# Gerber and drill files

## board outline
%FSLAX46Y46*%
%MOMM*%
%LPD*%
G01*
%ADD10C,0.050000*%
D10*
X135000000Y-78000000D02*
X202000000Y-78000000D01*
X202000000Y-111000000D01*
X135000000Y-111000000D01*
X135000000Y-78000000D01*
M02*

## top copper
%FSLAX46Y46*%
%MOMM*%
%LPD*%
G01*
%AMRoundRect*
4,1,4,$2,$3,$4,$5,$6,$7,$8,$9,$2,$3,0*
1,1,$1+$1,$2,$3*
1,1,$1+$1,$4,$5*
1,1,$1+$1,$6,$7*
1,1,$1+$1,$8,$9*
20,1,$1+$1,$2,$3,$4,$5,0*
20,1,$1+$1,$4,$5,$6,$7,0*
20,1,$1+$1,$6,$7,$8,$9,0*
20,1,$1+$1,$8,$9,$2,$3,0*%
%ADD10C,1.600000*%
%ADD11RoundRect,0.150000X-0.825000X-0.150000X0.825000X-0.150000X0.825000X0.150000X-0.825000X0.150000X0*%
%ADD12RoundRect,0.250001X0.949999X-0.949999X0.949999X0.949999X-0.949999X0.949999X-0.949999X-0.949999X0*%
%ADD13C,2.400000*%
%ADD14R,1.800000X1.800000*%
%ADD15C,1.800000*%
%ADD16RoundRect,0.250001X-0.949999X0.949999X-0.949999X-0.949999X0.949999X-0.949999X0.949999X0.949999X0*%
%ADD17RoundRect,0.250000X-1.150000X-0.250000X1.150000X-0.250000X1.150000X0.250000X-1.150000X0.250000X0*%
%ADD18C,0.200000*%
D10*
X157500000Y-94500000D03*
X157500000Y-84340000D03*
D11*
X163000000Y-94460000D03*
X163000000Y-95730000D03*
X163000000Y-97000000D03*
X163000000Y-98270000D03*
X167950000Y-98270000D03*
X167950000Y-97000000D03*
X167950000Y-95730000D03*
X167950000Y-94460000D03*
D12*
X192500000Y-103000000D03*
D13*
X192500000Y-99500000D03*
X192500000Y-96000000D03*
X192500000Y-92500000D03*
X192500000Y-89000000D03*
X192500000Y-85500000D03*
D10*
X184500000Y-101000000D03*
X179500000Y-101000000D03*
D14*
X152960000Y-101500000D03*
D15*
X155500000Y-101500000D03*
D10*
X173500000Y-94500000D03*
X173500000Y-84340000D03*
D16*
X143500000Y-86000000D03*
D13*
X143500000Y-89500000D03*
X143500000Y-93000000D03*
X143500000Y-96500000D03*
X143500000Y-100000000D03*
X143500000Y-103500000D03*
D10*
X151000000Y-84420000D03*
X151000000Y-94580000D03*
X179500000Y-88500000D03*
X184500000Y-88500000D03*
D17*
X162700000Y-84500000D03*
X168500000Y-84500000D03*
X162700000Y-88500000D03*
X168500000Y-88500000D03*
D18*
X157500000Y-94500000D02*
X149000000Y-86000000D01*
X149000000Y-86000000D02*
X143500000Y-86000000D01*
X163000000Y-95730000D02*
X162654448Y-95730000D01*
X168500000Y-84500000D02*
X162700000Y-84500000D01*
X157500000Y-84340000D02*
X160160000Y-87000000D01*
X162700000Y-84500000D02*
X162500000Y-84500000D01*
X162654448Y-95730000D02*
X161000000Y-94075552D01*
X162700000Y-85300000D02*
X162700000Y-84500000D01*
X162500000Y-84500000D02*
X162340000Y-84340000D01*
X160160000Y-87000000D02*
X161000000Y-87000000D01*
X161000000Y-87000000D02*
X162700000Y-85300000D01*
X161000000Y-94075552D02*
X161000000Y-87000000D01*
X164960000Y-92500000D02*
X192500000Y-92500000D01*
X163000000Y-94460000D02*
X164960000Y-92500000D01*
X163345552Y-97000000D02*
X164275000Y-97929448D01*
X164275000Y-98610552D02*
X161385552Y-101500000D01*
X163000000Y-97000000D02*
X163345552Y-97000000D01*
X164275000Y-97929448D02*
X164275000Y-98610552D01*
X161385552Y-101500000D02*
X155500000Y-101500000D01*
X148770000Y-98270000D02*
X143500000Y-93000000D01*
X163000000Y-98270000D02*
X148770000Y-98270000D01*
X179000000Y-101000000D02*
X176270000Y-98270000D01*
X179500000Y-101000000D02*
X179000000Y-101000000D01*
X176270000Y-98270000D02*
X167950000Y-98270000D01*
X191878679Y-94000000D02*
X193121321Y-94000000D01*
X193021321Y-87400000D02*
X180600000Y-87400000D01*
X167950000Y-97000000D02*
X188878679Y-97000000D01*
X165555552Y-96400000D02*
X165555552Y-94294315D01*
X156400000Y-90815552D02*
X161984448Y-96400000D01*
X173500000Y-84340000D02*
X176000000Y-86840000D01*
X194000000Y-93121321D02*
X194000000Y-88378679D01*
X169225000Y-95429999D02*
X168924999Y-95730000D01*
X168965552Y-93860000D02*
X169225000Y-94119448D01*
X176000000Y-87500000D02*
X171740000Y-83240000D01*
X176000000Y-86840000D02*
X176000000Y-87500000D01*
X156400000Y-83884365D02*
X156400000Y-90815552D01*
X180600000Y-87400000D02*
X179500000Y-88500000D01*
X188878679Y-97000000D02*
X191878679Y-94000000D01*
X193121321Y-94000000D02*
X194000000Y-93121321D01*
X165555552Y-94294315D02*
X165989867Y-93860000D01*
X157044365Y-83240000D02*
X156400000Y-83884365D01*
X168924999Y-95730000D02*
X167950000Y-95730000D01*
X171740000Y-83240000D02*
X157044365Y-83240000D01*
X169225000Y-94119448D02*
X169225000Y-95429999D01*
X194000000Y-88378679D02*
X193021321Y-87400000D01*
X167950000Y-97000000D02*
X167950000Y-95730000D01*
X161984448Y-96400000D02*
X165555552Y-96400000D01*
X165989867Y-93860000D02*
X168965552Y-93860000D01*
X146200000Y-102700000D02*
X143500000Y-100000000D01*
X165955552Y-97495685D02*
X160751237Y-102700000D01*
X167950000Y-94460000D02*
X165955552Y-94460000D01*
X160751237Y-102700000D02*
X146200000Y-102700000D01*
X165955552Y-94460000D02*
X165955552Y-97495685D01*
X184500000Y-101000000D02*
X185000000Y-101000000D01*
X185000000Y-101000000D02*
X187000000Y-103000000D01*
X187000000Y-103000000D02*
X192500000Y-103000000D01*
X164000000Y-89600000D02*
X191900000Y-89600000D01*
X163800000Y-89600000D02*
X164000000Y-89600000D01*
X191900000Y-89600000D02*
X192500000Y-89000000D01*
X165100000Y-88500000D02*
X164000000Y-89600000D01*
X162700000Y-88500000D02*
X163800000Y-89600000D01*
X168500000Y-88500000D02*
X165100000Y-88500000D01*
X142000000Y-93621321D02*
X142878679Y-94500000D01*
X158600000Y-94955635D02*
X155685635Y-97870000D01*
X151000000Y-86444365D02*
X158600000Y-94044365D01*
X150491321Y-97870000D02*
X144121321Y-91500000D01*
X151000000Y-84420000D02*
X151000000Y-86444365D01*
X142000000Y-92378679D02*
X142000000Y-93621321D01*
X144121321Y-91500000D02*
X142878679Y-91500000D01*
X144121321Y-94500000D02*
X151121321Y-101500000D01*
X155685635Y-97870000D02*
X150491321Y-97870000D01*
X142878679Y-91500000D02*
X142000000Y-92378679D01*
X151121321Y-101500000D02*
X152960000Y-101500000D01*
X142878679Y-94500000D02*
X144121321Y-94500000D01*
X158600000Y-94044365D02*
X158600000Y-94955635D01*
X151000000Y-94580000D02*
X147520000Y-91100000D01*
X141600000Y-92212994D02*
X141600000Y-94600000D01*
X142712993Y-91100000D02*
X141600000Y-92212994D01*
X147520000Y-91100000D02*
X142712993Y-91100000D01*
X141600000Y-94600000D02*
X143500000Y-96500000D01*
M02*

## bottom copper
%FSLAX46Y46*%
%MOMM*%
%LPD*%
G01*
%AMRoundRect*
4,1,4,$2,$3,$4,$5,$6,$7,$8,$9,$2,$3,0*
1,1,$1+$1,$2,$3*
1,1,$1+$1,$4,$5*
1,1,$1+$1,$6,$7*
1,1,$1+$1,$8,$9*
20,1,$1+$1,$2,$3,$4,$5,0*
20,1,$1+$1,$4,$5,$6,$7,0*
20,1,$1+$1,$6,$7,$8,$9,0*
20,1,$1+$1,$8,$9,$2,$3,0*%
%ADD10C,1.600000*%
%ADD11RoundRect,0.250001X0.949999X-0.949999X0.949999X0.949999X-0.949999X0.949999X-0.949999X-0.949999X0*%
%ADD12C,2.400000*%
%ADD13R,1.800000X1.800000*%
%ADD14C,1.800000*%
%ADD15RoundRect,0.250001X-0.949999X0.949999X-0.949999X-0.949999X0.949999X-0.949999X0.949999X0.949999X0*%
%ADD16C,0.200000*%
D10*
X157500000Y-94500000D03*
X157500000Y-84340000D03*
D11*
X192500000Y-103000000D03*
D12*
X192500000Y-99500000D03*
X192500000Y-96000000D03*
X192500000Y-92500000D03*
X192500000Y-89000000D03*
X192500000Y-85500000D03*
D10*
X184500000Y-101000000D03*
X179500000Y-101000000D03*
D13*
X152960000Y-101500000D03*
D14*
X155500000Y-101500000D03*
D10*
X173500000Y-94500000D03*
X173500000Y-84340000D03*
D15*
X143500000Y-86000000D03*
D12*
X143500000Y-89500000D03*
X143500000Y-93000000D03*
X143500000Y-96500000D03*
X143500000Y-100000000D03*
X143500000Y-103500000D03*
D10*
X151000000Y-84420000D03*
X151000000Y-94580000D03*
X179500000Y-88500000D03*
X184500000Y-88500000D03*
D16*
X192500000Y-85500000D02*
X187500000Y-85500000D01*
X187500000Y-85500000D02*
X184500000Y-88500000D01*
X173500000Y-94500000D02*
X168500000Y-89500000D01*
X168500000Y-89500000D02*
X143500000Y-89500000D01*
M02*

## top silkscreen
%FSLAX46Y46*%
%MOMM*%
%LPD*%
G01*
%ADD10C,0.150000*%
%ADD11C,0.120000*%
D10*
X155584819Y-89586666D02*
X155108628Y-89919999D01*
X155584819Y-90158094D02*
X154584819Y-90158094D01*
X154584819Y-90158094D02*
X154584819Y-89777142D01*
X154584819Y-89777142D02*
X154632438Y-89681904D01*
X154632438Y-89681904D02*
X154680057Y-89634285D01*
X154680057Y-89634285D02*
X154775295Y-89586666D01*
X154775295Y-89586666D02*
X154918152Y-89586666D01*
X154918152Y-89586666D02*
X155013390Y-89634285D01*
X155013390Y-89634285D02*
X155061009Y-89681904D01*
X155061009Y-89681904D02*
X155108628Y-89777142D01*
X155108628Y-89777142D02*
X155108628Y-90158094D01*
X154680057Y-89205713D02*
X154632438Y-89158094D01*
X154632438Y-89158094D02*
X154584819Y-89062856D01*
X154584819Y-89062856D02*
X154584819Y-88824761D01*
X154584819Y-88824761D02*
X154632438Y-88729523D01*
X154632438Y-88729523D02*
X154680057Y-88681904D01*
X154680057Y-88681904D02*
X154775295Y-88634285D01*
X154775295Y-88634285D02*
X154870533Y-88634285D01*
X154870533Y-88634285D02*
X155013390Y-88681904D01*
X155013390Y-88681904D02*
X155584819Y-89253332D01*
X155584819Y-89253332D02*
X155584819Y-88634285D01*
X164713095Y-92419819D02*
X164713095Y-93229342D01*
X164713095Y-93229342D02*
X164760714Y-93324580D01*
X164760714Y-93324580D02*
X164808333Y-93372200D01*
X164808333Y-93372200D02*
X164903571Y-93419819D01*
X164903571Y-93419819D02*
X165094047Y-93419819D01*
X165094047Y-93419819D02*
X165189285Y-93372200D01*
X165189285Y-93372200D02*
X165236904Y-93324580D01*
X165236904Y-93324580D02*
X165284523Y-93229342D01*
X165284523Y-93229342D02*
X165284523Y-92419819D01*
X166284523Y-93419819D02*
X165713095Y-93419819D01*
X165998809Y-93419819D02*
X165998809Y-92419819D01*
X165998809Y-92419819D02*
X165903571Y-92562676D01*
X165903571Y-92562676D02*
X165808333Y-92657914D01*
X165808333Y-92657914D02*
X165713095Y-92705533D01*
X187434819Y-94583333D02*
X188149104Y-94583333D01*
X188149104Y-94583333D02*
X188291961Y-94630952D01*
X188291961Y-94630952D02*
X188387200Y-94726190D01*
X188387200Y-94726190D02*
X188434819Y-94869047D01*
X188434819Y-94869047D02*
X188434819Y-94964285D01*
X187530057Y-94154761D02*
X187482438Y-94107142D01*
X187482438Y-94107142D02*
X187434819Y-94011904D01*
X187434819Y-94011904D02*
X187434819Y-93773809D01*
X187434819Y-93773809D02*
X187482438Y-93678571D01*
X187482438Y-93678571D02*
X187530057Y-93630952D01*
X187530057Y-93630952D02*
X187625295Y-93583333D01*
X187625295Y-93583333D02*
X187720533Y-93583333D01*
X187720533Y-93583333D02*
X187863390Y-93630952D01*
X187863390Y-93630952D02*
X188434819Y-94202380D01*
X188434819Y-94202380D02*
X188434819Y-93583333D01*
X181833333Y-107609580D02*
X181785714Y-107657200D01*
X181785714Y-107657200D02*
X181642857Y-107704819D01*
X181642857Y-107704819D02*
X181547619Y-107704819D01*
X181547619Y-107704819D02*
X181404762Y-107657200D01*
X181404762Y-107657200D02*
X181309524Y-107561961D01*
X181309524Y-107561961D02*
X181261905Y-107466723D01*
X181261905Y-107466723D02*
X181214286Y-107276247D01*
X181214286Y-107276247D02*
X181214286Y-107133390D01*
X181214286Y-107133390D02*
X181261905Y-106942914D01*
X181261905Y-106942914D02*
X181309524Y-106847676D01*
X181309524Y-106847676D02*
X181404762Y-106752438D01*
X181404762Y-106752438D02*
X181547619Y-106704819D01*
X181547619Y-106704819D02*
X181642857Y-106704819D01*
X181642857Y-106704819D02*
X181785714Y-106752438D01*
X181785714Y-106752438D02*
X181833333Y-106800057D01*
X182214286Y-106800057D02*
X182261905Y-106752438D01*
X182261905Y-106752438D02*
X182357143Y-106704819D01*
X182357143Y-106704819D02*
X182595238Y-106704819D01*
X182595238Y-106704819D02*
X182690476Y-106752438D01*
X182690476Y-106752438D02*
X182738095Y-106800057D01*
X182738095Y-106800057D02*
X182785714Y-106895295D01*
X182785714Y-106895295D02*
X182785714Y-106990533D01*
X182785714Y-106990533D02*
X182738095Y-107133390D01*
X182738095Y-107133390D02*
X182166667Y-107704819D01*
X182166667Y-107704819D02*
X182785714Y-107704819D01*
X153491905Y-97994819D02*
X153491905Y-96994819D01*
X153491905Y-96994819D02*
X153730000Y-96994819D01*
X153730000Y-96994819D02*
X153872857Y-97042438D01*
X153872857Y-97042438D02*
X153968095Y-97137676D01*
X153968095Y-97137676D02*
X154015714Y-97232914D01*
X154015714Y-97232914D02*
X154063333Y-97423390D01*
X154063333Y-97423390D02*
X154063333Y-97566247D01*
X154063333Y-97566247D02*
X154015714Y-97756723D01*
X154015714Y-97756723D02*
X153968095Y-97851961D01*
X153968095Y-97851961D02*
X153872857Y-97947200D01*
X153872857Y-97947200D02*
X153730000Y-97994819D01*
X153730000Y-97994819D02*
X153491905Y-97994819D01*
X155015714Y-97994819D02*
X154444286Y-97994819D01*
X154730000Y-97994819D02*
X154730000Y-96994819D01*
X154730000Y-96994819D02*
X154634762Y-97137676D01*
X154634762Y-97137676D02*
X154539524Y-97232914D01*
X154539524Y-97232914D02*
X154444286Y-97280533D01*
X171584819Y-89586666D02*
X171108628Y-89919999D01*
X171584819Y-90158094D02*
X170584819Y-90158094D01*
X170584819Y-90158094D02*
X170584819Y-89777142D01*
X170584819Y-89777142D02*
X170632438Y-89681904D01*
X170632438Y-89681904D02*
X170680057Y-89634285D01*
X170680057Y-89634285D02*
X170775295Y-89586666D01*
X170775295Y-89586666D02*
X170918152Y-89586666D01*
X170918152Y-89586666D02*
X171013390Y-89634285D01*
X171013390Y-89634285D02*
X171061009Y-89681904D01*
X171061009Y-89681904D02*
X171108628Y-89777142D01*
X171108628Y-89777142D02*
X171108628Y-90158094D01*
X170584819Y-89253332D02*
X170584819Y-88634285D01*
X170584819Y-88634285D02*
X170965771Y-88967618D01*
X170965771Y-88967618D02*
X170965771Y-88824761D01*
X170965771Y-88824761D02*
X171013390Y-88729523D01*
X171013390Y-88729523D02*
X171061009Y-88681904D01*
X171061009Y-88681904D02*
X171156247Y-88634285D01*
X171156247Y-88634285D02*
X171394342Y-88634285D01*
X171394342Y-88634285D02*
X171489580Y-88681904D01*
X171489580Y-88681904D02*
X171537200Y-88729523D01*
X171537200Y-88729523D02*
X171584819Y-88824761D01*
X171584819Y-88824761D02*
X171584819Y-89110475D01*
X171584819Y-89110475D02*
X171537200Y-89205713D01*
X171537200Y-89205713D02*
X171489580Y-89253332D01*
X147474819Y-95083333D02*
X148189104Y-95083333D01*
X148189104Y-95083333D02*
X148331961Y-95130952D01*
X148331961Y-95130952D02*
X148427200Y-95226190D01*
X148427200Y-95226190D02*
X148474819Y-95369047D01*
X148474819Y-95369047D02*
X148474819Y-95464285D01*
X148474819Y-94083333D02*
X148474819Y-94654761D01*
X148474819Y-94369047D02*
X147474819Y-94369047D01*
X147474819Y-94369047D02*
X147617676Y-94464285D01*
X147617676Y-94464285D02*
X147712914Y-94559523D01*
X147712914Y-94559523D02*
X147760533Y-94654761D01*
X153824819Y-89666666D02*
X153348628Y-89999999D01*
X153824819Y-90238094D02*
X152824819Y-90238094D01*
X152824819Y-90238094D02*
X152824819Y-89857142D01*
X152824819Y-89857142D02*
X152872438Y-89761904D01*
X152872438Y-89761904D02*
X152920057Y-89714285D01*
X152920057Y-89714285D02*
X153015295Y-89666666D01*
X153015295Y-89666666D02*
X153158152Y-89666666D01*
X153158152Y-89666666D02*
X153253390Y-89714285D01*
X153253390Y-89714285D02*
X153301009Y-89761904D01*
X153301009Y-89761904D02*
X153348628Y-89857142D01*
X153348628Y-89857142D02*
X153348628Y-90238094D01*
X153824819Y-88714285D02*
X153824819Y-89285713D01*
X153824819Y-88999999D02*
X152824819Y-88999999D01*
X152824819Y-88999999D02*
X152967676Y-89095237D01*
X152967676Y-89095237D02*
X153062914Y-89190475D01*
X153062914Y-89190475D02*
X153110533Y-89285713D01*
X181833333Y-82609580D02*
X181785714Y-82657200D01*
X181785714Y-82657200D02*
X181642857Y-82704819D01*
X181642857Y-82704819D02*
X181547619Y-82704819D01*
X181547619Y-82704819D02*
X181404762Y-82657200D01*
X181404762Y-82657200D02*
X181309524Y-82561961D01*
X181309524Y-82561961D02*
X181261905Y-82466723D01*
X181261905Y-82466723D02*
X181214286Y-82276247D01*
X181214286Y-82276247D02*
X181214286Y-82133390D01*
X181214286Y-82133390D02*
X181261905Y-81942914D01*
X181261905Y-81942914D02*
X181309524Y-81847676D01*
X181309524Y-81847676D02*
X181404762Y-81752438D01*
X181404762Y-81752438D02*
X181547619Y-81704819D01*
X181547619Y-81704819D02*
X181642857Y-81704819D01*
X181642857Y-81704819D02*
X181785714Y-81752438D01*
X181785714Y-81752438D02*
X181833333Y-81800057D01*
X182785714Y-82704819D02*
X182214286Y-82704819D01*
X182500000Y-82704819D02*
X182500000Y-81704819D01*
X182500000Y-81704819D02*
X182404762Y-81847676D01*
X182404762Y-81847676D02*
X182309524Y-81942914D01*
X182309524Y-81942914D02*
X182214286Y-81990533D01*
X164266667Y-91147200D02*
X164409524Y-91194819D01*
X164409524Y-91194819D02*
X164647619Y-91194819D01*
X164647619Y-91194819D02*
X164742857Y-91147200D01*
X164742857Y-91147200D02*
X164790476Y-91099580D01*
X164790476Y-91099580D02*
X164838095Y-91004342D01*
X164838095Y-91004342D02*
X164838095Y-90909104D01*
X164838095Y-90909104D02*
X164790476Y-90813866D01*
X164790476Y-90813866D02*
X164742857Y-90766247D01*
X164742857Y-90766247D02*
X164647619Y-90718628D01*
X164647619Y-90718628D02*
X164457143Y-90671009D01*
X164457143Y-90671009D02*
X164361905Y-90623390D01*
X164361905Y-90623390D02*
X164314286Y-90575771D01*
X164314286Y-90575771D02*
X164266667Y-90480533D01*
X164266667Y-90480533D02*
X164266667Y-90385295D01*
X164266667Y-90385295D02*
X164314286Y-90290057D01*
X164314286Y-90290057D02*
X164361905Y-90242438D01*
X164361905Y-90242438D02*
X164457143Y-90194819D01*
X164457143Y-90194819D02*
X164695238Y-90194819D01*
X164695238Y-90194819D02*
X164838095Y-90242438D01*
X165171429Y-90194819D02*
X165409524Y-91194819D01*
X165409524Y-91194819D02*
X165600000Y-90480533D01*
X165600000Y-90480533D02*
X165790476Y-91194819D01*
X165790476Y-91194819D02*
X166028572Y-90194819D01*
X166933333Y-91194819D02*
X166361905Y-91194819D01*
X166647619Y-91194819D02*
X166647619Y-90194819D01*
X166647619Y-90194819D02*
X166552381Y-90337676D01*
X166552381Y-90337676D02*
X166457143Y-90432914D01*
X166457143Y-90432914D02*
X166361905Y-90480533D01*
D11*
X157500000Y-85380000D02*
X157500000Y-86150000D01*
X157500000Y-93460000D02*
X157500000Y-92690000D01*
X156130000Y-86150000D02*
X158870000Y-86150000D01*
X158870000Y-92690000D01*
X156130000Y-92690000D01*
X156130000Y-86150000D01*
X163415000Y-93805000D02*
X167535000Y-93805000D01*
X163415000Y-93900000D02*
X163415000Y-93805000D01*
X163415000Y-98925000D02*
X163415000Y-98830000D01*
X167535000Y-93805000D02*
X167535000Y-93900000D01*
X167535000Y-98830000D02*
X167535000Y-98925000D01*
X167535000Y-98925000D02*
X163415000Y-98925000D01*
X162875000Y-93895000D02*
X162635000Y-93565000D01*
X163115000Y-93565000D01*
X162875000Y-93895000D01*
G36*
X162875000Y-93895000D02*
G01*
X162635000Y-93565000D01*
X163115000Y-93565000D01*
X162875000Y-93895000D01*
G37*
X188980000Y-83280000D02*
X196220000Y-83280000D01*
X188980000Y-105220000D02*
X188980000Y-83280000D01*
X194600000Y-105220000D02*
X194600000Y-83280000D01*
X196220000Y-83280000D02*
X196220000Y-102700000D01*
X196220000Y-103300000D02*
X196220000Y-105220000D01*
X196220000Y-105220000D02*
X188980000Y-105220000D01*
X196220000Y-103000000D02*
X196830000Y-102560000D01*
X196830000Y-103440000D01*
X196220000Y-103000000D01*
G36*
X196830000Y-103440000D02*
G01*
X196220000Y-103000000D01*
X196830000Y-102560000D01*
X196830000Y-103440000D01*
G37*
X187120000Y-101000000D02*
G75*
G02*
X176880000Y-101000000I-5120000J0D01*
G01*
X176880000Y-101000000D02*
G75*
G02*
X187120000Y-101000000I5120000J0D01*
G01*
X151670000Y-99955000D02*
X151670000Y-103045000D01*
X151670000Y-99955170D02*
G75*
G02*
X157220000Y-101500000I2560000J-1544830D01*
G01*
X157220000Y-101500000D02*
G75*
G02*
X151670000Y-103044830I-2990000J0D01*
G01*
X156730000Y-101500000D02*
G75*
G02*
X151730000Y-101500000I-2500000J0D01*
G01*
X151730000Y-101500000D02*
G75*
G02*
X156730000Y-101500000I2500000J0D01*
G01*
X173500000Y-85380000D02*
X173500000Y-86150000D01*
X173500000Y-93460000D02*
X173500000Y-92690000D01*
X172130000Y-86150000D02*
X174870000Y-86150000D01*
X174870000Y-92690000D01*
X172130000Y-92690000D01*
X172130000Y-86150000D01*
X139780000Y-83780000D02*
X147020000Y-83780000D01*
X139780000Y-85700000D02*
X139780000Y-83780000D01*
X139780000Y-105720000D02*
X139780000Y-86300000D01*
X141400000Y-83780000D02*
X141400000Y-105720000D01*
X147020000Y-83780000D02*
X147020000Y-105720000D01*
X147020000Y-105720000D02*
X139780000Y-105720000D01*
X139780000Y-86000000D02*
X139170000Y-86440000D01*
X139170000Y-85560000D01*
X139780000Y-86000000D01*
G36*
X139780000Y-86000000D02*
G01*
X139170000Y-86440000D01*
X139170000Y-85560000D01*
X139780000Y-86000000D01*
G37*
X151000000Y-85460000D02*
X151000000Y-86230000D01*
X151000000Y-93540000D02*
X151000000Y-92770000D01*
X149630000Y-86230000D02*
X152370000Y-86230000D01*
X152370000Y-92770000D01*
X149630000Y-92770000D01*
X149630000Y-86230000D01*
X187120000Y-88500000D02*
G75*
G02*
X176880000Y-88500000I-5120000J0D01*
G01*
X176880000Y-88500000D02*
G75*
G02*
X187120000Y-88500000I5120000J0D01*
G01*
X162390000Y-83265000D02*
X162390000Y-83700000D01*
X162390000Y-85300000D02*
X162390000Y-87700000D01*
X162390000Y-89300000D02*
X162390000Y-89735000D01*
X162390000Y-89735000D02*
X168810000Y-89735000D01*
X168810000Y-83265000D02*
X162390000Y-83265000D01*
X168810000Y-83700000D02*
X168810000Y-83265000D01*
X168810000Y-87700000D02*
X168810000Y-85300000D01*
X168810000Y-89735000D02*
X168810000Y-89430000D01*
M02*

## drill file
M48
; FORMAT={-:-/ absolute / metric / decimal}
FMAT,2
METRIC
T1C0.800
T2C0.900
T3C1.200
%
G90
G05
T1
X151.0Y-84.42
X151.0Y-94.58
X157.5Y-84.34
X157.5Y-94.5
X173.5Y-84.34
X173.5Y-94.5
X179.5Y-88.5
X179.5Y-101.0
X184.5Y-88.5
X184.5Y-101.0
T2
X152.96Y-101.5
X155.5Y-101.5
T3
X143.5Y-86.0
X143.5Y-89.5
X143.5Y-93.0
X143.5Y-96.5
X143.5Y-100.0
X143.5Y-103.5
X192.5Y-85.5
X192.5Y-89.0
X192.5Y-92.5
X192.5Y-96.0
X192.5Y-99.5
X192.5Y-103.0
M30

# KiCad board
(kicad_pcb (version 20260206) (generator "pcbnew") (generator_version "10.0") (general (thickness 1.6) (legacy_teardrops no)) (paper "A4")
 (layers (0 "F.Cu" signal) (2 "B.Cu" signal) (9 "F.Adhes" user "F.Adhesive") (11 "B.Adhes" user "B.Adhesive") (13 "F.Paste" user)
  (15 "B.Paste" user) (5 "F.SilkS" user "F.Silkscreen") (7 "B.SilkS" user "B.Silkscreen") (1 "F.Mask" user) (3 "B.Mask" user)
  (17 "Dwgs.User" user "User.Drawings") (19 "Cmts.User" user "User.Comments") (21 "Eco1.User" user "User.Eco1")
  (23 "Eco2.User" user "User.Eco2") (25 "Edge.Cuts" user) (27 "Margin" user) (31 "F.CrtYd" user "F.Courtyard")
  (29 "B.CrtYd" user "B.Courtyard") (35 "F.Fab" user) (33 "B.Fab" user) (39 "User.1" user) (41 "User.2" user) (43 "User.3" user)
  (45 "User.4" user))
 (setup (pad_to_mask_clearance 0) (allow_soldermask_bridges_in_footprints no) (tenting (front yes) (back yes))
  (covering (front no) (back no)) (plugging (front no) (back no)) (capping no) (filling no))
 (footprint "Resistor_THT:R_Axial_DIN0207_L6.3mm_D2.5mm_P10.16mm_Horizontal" (layer "F.Cu") (at 157.5 94.5 90)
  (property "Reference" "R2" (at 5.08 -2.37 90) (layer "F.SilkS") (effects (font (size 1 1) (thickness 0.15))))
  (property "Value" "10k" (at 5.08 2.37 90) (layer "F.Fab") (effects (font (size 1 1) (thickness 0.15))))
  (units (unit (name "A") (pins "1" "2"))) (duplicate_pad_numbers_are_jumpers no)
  (fp_line (start 9.12 0) (end 8.35 0) (stroke (width 0.12) (type solid)) (layer "F.SilkS"))
  (fp_line (start 1.04 0) (end 1.81 0) (stroke (width 0.12) (type solid)) (layer "F.SilkS"))
  (fp_rect (start 1.81 -1.37) (end 8.35 1.37) (stroke (width 0.12) (type solid)) (fill no) (layer "F.SilkS"))
  (pad "1" thru_hole circle (at 0 0 90) (size 1.6 1.6) (drill 0.8) (layers "*.Cu" "*.Mask") (remove_unused_layers no) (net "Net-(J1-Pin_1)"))
  (pad "2" thru_hole circle (at 10.16 0 90) (size 1.6 1.6) (drill 0.8) (layers "*.Cu" "*.Mask") (remove_unused_layers no)
   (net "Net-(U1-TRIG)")))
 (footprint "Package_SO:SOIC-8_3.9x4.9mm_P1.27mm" (layer "F.Cu") (at 165.475 96.365)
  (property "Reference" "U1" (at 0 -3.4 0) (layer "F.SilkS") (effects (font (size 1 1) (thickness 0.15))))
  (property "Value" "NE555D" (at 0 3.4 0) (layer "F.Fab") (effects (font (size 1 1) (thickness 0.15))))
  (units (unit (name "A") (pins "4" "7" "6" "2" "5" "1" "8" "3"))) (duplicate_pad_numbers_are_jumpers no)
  (fp_line (start -2.06 -2.56) (end 2.06 -2.56) (stroke (width 0.12) (type solid)) (layer "F.SilkS"))
  (fp_line (start -2.06 -2.465) (end -2.06 -2.56) (stroke (width 0.12) (type solid)) (layer "F.SilkS"))
  (fp_line (start -2.06 2.56) (end -2.06 2.465) (stroke (width 0.12) (type solid)) (layer "F.SilkS"))
  (fp_line (start 2.06 -2.56) (end 2.06 -2.465) (stroke (width 0.12) (type solid)) (layer "F.SilkS"))
  (fp_line (start 2.06 2.465) (end 2.06 2.56) (stroke (width 0.12) (type solid)) (layer "F.SilkS"))
  (fp_line (start 2.06 2.56) (end -2.06 2.56) (stroke (width 0.12) (type solid)) (layer "F.SilkS"))
  (fp_poly (pts (xy -2.6 -2.47) (xy -2.84 -2.8) (xy -2.36 -2.8)) (stroke (width 0.12) (type solid)) (fill yes) (layer "F.SilkS"))
  (pad "1" smd roundrect (at -2.475 -1.905) (size 1.95 0.6) (layers "F.Cu" "F.Mask" "F.Paste") (roundrect_rratio 0.25) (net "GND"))
  (pad "2" smd roundrect (at -2.475 -0.635) (size 1.95 0.6) (layers "F.Cu" "F.Mask" "F.Paste") (roundrect_rratio 0.25) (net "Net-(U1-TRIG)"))
  (pad "3" smd roundrect (at -2.475 0.635) (size 1.95 0.6) (layers "F.Cu" "F.Mask" "F.Paste") (roundrect_rratio 0.25) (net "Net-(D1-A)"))
  (pad "4" smd roundrect (at -2.475 1.905) (size 1.95 0.6) (layers "F.Cu" "F.Mask" "F.Paste") (roundrect_rratio 0.25) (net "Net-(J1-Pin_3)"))
  (pad "5" smd roundrect (at 2.475 1.905) (size 1.95 0.6) (layers "F.Cu" "F.Mask" "F.Paste") (roundrect_rratio 0.25) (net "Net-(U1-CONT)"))
  (pad "6" smd roundrect (at 2.475 0.635) (size 1.95 0.6) (layers "F.Cu" "F.Mask" "F.Paste") (roundrect_rratio 0.25) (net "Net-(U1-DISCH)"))
  (pad "7" smd roundrect (at 2.475 -0.635) (size 1.95 0.6) (layers "F.Cu" "F.Mask" "F.Paste") (roundrect_rratio 0.25) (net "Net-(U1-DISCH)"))
  (pad "8" smd roundrect (at 2.475 -1.905) (size 1.95 0.6) (layers "F.Cu" "F.Mask" "F.Paste") (roundrect_rratio 0.25) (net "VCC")))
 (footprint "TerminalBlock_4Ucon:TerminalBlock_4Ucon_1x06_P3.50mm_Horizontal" (layer "F.Cu") (at 192.5 103 90)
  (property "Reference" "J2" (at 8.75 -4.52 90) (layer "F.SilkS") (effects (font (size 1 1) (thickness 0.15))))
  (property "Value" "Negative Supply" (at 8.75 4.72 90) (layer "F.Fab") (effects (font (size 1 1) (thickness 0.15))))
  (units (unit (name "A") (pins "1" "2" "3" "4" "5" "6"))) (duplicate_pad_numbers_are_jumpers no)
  (fp_line (start 19.72 -3.52) (end 19.72 3.72) (stroke (width 0.12) (type solid)) (layer "F.SilkS"))
  (fp_line (start -2.22 -3.52) (end 19.72 -3.52) (stroke (width 0.12) (type solid)) (layer "F.SilkS"))
  (fp_line (start -2.22 2.1) (end 19.72 2.1) (stroke (width 0.12) (type solid)) (layer "F.SilkS"))
  (fp_line (start 19.72 3.72) (end 0.3 3.72) (stroke (width 0.12) (type solid)) (layer "F.SilkS"))
  (fp_line (start -0.3 3.72) (end -2.22 3.72) (stroke (width 0.12) (type solid)) (layer "F.SilkS"))
  (fp_line (start -2.22 3.72) (end -2.22 -3.52) (stroke (width 0.12) (type solid)) (layer "F.SilkS"))
  (fp_poly (pts (xy 0 3.72) (xy 0.44 4.33) (xy -0.44 4.33)) (stroke (width 0.12) (type solid)) (fill yes) (layer "F.SilkS"))
  (pad "1" thru_hole roundrect (at 0 0 90) (size 2.4 2.4) (drill 1.2) (layers "*.Cu" "*.Mask") (remove_unused_layers no)
   (roundrect_rratio 0.104167) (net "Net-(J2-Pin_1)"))
  (pad "2" thru_hole circle (at 3.5 0 90) (size 2.4 2.4) (drill 1.2) (layers "*.Cu" "*.Mask") (remove_unused_layers no)
   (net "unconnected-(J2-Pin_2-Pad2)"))
  (pad "3" thru_hole circle (at 7 0 90) (size 2.4 2.4) (drill 1.2) (layers "*.Cu" "*.Mask") (remove_unused_layers no)
   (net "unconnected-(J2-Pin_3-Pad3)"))
  (pad "4" thru_hole circle (at 10.5 0 90) (size 2.4 2.4) (drill 1.2) (layers "*.Cu" "*.Mask") (remove_unused_layers no) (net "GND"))
  (pad "5" thru_hole circle (at 14 0 90) (size 2.4 2.4) (drill 1.2) (layers "*.Cu" "*.Mask") (remove_unused_layers no)
   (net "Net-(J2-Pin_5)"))
  (pad "6" thru_hole circle (at 17.5 0 90) (size 2.4 2.4) (drill 1.2) (layers "*.Cu" "*.Mask") (remove_unused_layers no)
   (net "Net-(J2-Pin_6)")))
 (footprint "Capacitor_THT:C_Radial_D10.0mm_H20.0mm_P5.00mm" (layer "F.Cu") (at 184.5 101 180)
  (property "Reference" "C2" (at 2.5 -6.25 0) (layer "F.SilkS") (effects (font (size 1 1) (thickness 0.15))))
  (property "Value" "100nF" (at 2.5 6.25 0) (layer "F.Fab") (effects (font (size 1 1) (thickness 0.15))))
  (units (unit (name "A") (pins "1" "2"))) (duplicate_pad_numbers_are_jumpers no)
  (fp_circle (center 2.5 0) (end 7.62 0) (stroke (width 0.12) (type solid)) (fill no) (layer "F.SilkS"))
  (pad "1" thru_hole circle (at 0 0 180) (size 1.6 1.6) (drill 0.8) (layers "*.Cu" "*.Mask") (remove_unused_layers no)
   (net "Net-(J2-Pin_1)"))
  (pad "2" thru_hole circle (at 5 0 180) (size 1.6 1.6) (drill 0.8) (layers "*.Cu" "*.Mask") (remove_unused_layers no) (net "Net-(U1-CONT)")))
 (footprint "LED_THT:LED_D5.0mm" (layer "F.Cu") (at 152.96 101.5)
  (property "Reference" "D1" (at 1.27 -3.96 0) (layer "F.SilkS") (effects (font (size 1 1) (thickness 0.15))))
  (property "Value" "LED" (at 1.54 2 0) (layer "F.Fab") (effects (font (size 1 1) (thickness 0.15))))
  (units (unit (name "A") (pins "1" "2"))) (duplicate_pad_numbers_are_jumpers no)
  (fp_line (start -1.29 -1.545) (end -1.29 1.545) (stroke (width 0.12) (type solid)) (layer "F.SilkS"))
  (fp_arc (start -1.29 -1.54483) (mid 2.071779 -2.880495) (end 4.26 0) (stroke (width 0.12) (type solid)) (layer "F.SilkS"))
  (fp_arc (start 4.26 0) (mid 2.071779 2.880495) (end -1.29 1.54483) (stroke (width 0.12) (type solid)) (layer "F.SilkS"))
  (fp_circle (center 1.27 0) (end 3.77 0) (stroke (width 0.12) (type solid)) (fill no) (layer "F.SilkS"))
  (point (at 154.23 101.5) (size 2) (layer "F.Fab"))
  (pad "1" thru_hole rect (at 0 0) (size 1.8 1.8) (drill 0.9) (layers "*.Cu" "*.Mask") (remove_unused_layers no) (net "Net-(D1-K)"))
  (pad "2" thru_hole circle (at 2.54 0) (size 1.8 1.8) (drill 0.9) (layers "*.Cu" "*.Mask") (remove_unused_layers no) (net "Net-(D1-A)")))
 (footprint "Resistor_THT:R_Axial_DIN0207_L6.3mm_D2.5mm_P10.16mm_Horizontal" (layer "F.Cu") (at 173.5 94.5 90)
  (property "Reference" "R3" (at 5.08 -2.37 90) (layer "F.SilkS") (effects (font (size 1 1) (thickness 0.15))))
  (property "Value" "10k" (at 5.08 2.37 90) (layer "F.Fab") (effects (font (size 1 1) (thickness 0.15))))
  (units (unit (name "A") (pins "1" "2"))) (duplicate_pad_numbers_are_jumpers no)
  (fp_line (start 9.12 0) (end 8.35 0) (stroke (width 0.12) (type solid)) (layer "F.SilkS"))
  (fp_line (start 1.04 0) (end 1.81 0) (stroke (width 0.12) (type solid)) (layer "F.SilkS"))
  (fp_rect (start 1.81 -1.37) (end 8.35 1.37) (stroke (width 0.12) (type solid)) (fill no) (layer "F.SilkS"))
  (pad "1" thru_hole circle (at 0 0 90) (size 1.6 1.6) (drill 0.8) (layers "*.Cu" "*.Mask") (remove_unused_layers no) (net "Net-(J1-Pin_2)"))
  (pad "2" thru_hole circle (at 10.16 0 90) (size 1.6 1.6) (drill 0.8) (layers "*.Cu" "*.Mask") (remove_unused_layers no)
   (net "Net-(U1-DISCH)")))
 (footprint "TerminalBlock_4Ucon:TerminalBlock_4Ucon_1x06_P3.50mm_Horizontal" (layer "F.Cu") (at 143.5 86 -90)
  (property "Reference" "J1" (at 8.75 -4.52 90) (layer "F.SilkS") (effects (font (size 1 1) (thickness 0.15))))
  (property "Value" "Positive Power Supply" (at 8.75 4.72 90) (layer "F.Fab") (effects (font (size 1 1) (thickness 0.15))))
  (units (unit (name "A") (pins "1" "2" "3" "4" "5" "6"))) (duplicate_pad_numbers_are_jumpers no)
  (fp_line (start -2.22 3.72) (end -2.22 -3.52) (stroke (width 0.12) (type solid)) (layer "F.SilkS"))
  (fp_line (start -0.3 3.72) (end -2.22 3.72) (stroke (width 0.12) (type solid)) (layer "F.SilkS"))
  (fp_line (start 19.72 3.72) (end 0.3 3.72) (stroke (width 0.12) (type solid)) (layer "F.SilkS"))
  (fp_line (start -2.22 2.1) (end 19.72 2.1) (stroke (width 0.12) (type solid)) (layer "F.SilkS"))
  (fp_line (start -2.22 -3.52) (end 19.72 -3.52) (stroke (width 0.12) (type solid)) (layer "F.SilkS"))
  (fp_line (start 19.72 -3.52) (end 19.72 3.72) (stroke (width 0.12) (type solid)) (layer "F.SilkS"))
  (fp_poly (pts (xy 0 3.72) (xy 0.44 4.33) (xy -0.44 4.33)) (stroke (width 0.12) (type solid)) (fill yes) (layer "F.SilkS"))
  (pad "1" thru_hole roundrect (at 0 0 270) (size 2.4 2.4) (drill 1.2) (layers "*.Cu" "*.Mask") (remove_unused_layers no)
   (roundrect_rratio 0.104167) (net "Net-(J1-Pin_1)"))
  (pad "2" thru_hole circle (at 3.5 0 270) (size 2.4 2.4) (drill 1.2) (layers "*.Cu" "*.Mask") (remove_unused_layers no)
   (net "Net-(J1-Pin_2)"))
  (pad "3" thru_hole circle (at 7 0 270) (size 2.4 2.4) (drill 1.2) (layers "*.Cu" "*.Mask") (remove_unused_layers no)
   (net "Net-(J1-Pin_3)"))
  (pad "4" thru_hole circle (at 10.5 0 270) (size 2.4 2.4) (drill 1.2) (layers "*.Cu" "*.Mask") (remove_unused_layers no)
   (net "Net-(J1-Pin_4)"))
  (pad "5" thru_hole circle (at 14 0 270) (size 2.4 2.4) (drill 1.2) (layers "*.Cu" "*.Mask") (remove_unused_layers no) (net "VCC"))
  (pad "6" thru_hole circle (at 17.5 0 270) (size 2.4 2.4) (drill 1.2) (layers "*.Cu" "*.Mask") (remove_unused_layers no)
   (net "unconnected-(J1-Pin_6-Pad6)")))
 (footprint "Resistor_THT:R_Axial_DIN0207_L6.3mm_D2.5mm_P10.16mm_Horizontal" (layer "F.Cu") (at 151 84.42 -90)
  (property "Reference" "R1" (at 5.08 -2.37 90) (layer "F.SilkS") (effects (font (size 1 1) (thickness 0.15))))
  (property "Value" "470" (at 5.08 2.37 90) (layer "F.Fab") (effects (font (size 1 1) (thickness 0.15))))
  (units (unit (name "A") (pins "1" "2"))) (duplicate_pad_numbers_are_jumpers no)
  (fp_line (start 1.04 0) (end 1.81 0) (stroke (width 0.12) (type solid)) (layer "F.SilkS"))
  (fp_line (start 9.12 0) (end 8.35 0) (stroke (width 0.12) (type solid)) (layer "F.SilkS"))
  (fp_rect (start 1.81 -1.37) (end 8.35 1.37) (stroke (width 0.12) (type solid)) (fill no) (layer "F.SilkS"))
  (pad "1" thru_hole circle (at 0 0 270) (size 1.6 1.6) (drill 0.8) (layers "*.Cu" "*.Mask") (remove_unused_layers no) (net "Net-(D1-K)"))
  (pad "2" thru_hole circle (at 10.16 0 270) (size 1.6 1.6) (drill 0.8) (layers "*.Cu" "*.Mask") (remove_unused_layers no)
   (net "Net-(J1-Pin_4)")))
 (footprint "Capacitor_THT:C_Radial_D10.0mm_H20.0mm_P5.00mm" (layer "F.Cu") (at 179.5 88.5)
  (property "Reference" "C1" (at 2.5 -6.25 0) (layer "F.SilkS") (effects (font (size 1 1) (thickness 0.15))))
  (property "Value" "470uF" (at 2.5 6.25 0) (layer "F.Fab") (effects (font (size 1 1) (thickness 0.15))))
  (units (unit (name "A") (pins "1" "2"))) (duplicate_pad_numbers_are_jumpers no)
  (fp_circle (center 2.5 0) (end 7.62 0) (stroke (width 0.12) (type solid)) (fill no) (layer "F.SilkS"))
  (pad "1" thru_hole circle (at 0 0) (size 1.6 1.6) (drill 0.8) (layers "*.Cu" "*.Mask") (remove_unused_layers no) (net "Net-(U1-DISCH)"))
  (pad "2" thru_hole circle (at 5 0) (size 1.6 1.6) (drill 0.8) (layers "*.Cu" "*.Mask") (remove_unused_layers no) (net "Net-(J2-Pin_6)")))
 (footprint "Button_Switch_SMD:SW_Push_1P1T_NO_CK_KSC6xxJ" (layer "F.Cu") (at 165.6 86.5)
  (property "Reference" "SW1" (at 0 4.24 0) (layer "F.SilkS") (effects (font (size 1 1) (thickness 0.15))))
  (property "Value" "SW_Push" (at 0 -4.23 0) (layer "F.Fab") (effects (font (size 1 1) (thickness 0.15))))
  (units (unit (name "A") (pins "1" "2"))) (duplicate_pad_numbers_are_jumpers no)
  (fp_line (start -3.21 -3.235) (end -3.21 -2.8) (stroke (width 0.12) (type solid)) (layer "F.SilkS"))
  (fp_line (start -3.21 -1.2) (end -3.21 1.2) (stroke (width 0.12) (type solid)) (layer "F.SilkS"))
  (fp_line (start -3.21 2.8) (end -3.21 3.235) (stroke (width 0.12) (type solid)) (layer "F.SilkS"))
  (fp_line (start -3.21 3.235) (end 3.21 3.235) (stroke (width 0.12) (type solid)) (layer "F.SilkS"))
  (fp_line (start 3.21 -3.235) (end -3.21 -3.235) (stroke (width 0.12) (type solid)) (layer "F.SilkS"))
  (fp_line (start 3.21 -2.8) (end 3.21 -3.235) (stroke (width 0.12) (type solid)) (layer "F.SilkS"))
  (fp_line (start 3.21 1.2) (end 3.21 -1.2) (stroke (width 0.12) (type solid)) (layer "F.SilkS"))
  (fp_line (start 3.21 3.235) (end 3.21 2.93) (stroke (width 0.12) (type solid)) (layer "F.SilkS"))
  (pad "1" smd roundrect (at -2.9 -2) (size 2.8 1) (layers "F.Cu" "F.Mask" "F.Paste") (roundrect_rratio 0.25) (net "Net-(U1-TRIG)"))
  (pad "1" smd roundrect (at 2.9 -2) (size 2.8 1) (layers "F.Cu" "F.Mask" "F.Paste") (roundrect_rratio 0.25) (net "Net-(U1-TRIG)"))
  (pad "2" smd roundrect (at -2.9 2) (size 2.8 1) (layers "F.Cu" "F.Mask" "F.Paste") (roundrect_rratio 0.25) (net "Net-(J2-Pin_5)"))
  (pad "2" smd roundrect (at 2.9 2) (size 2.8 1) (layers "F.Cu" "F.Mask" "F.Paste") (roundrect_rratio 0.25) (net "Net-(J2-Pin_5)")))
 (gr_rect (start 135 78) (end 202 111) (stroke (width 0.05) (type solid)) (fill no) (layer "Edge.Cuts"))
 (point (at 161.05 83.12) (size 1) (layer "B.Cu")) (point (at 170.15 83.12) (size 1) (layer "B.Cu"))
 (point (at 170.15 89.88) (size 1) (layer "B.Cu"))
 (segment (start 157.5 94.5) (end 149 86) (width 0.2) (layer "F.Cu") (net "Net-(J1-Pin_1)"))
 (segment (start 149 86) (end 143.5 86) (width 0.2) (layer "F.Cu") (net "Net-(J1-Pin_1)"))
 (segment (start 163 95.73) (end 162.654448 95.73) (width 0.2) (layer "F.Cu") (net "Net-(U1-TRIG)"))
 (segment (start 168.5 84.5) (end 162.7 84.5) (width 0.2) (layer "F.Cu") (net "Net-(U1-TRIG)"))
 (segment (start 157.5 84.34) (end 160.16 87) (width 0.2) (layer "F.Cu") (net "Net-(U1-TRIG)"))
 (segment (start 162.7 84.5) (end 162.5 84.5) (width 0.2) (layer "F.Cu") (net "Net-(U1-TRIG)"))
 (segment (start 162.654448 95.73) (end 161 94.075552) (width 0.2) (layer "F.Cu") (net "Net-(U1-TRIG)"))
 (segment (start 162.7 85.3) (end 162.7 84.5) (width 0.2) (layer "F.Cu") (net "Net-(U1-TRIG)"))
 (segment (start 162.5 84.5) (end 162.34 84.34) (width 0.2) (layer "F.Cu") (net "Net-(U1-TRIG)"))
 (segment (start 160.16 87) (end 161 87) (width 0.2) (layer "F.Cu") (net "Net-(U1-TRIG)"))
 (segment (start 161 87) (end 162.7 85.3) (width 0.2) (layer "F.Cu") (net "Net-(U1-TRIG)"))
 (segment (start 161 94.075552) (end 161 87) (width 0.2) (layer "F.Cu") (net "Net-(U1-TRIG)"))
 (segment (start 164.96 92.5) (end 192.5 92.5) (width 0.2) (layer "F.Cu") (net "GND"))
 (segment (start 163 94.46) (end 164.96 92.5) (width 0.2) (layer "F.Cu") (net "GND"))
 (segment (start 163.345552 97) (end 164.275 97.929448) (width 0.2) (layer "F.Cu") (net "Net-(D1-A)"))
 (segment (start 164.275 98.610552) (end 161.385552 101.5) (width 0.2) (layer "F.Cu") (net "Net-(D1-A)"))
 (segment (start 163 97) (end 163.345552 97) (width 0.2) (layer "F.Cu") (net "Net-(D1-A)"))
 (segment (start 164.275 97.929448) (end 164.275 98.610552) (width 0.2) (layer "F.Cu") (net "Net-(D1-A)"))
 (segment (start 161.385552 101.5) (end 155.5 101.5) (width 0.2) (layer "F.Cu") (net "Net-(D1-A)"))
 (segment (start 148.77 98.27) (end 143.5 93) (width 0.2) (layer "F.Cu") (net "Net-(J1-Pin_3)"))
 (segment (start 163 98.27) (end 148.77 98.27) (width 0.2) (layer "F.Cu") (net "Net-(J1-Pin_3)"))
 (segment (start 179 101) (end 176.27 98.27) (width 0.2) (layer "F.Cu") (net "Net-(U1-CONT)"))
 (segment (start 179.5 101) (end 179 101) (width 0.2) (layer "F.Cu") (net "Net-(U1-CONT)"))
 (segment (start 176.27 98.27) (end 167.95 98.27) (width 0.2) (layer "F.Cu") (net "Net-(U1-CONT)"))
 (segment (start 191.878679 94) (end 193.121321 94) (width 0.2) (layer "F.Cu") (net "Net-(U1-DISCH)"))
 (segment (start 193.021321 87.4) (end 180.6 87.4) (width 0.2) (layer "F.Cu") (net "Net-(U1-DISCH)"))
 (segment (start 167.95 97) (end 188.878679 97) (width 0.2) (layer "F.Cu") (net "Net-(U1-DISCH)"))
 (segment (start 165.555552 96.4) (end 165.555552 94.294315) (width 0.2) (layer "F.Cu") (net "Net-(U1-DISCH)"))
 (segment (start 156.4 90.815552) (end 161.984448 96.4) (width 0.2) (layer "F.Cu") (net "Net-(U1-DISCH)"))
 (segment (start 173.5 84.34) (end 176 86.84) (width 0.2) (layer "F.Cu") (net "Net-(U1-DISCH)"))
 (segment (start 194 93.121321) (end 194 88.378679) (width 0.2) (layer "F.Cu") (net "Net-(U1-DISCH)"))
 (segment (start 169.225 95.429999) (end 168.924999 95.73) (width 0.2) (layer "F.Cu") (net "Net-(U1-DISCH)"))
 (segment (start 168.965552 93.86) (end 169.225 94.119448) (width 0.2) (layer "F.Cu") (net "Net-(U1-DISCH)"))
 (segment (start 176 87.5) (end 171.74 83.24) (width 0.2) (layer "F.Cu") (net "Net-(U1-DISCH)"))
 (segment (start 176 86.84) (end 176 87.5) (width 0.2) (layer "F.Cu") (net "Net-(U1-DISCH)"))
 (segment (start 156.4 83.884365) (end 156.4 90.815552) (width 0.2) (layer "F.Cu") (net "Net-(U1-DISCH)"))
 (segment (start 180.6 87.4) (end 179.5 88.5) (width 0.2) (layer "F.Cu") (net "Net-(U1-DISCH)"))
 (segment (start 188.878679 97) (end 191.878679 94) (width 0.2) (layer "F.Cu") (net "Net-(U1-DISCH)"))
 (segment (start 193.121321 94) (end 194 93.121321) (width 0.2) (layer "F.Cu") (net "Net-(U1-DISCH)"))
 (segment (start 165.555552 94.294315) (end 165.989867 93.86) (width 0.2) (layer "F.Cu") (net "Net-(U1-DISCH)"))
 (segment (start 157.044365 83.24) (end 156.4 83.884365) (width 0.2) (layer "F.Cu") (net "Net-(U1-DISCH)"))
 (segment (start 168.924999 95.73) (end 167.95 95.73) (width 0.2) (layer "F.Cu") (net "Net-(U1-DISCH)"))
 (segment (start 171.74 83.24) (end 157.044365 83.24) (width 0.2) (layer "F.Cu") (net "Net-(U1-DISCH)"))
 (segment (start 169.225 94.119448) (end 169.225 95.429999) (width 0.2) (layer "F.Cu") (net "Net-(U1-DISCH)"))
 (segment (start 194 88.378679) (end 193.021321 87.4) (width 0.2) (layer "F.Cu") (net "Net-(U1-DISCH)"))
 (segment (start 167.95 97) (end 167.95 95.73) (width 0.2) (layer "F.Cu") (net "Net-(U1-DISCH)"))
 (segment (start 161.984448 96.4) (end 165.555552 96.4) (width 0.2) (layer "F.Cu") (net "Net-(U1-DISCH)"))
 (segment (start 165.989867 93.86) (end 168.965552 93.86) (width 0.2) (layer "F.Cu") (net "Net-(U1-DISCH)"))
 (segment (start 146.2 102.7) (end 143.5 100) (width 0.2) (layer "F.Cu") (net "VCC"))
 (segment (start 165.955552 97.495685) (end 160.751237 102.7) (width 0.2) (layer "F.Cu") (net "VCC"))
 (segment (start 167.95 94.46) (end 165.955552 94.46) (width 0.2) (layer "F.Cu") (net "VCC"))
 (segment (start 160.751237 102.7) (end 146.2 102.7) (width 0.2) (layer "F.Cu") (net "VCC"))
 (segment (start 165.955552 94.46) (end 165.955552 97.495685) (width 0.2) (layer "F.Cu") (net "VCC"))
 (segment (start 184.5 101) (end 185 101) (width 0.2) (layer "F.Cu") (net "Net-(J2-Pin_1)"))
 (segment (start 185 101) (end 187 103) (width 0.2) (layer "F.Cu") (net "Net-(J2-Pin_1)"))
 (segment (start 187 103) (end 192.5 103) (width 0.2) (layer "F.Cu") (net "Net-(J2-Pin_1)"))
 (segment (start 164 89.6) (end 191.9 89.6) (width 0.2) (layer "F.Cu") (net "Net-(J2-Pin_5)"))
 (segment (start 163.8 89.6) (end 164 89.6) (width 0.2) (layer "F.Cu") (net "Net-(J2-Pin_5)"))
 (segment (start 191.9 89.6) (end 192.5 89) (width 0.2) (layer "F.Cu") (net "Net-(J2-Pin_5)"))
 (segment (start 165.1 88.5) (end 164 89.6) (width 0.2) (layer "F.Cu") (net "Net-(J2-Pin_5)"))
 (segment (start 162.7 88.5) (end 163.8 89.6) (width 0.2) (layer "F.Cu") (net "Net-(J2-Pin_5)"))
 (segment (start 168.5 88.5) (end 165.1 88.5) (width 0.2) (layer "F.Cu") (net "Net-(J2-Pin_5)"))
 (segment (start 192.5 85.5) (end 187.5 85.5) (width 0.2) (layer "B.Cu") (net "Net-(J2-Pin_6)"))
 (segment (start 187.5 85.5) (end 184.5 88.5) (width 0.2) (layer "B.Cu") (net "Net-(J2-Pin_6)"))
 (segment (start 142 93.621321) (end 142.878679 94.5) (width 0.2) (layer "F.Cu") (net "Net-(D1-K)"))
 (segment (start 158.6 94.955635) (end 155.685635 97.87) (width 0.2) (layer "F.Cu") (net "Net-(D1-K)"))
 (segment (start 151 86.444365) (end 158.6 94.044365) (width 0.2) (layer "F.Cu") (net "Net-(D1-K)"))
 (segment (start 150.491321 97.87) (end 144.121321 91.5) (width 0.2) (layer "F.Cu") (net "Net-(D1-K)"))
 (segment (start 151 84.42) (end 151 86.444365) (width 0.2) (layer "F.Cu") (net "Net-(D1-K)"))
 (segment (start 142 92.378679) (end 142 93.621321) (width 0.2) (layer "F.Cu") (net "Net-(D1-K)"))
 (segment (start 144.121321 91.5) (end 142.878679 91.5) (width 0.2) (layer "F.Cu") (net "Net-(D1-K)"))
 (segment (start 144.121321 94.5) (end 151.121321 101.5) (width 0.2) (layer "F.Cu") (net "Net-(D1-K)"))
 (segment (start 155.685635 97.87) (end 150.491321 97.87) (width 0.2) (layer "F.Cu") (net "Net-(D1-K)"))
 (segment (start 142.878679 91.5) (end 142 92.378679) (width 0.2) (layer "F.Cu") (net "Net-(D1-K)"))
 (segment (start 151.121321 101.5) (end 152.96 101.5) (width 0.2) (layer "F.Cu") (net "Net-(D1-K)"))
 (segment (start 142.878679 94.5) (end 144.121321 94.5) (width 0.2) (layer "F.Cu") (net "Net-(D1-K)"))
 (segment (start 158.6 94.044365) (end 158.6 94.955635) (width 0.2) (layer "F.Cu") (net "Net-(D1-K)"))
 (segment (start 173.5 94.5) (end 168.5 89.5) (width 0.2) (layer "B.Cu") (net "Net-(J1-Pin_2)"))
 (segment (start 168.5 89.5) (end 143.5 89.5) (width 0.2) (layer "B.Cu") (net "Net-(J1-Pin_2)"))
 (segment (start 151 94.58) (end 147.52 91.1) (width 0.2) (layer "F.Cu") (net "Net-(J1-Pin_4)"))
 (segment (start 141.6 92.212994) (end 141.6 94.6) (width 0.2) (layer "F.Cu") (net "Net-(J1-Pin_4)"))
 (segment (start 142.712993 91.1) (end 141.6 92.212994) (width 0.2) (layer "F.Cu") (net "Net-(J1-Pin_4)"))
 (segment (start 147.52 91.1) (end 142.712993 91.1) (width 0.2) (layer "F.Cu") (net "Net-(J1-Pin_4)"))
 (segment (start 141.6 94.6) (end 143.5 96.5) (width 0.2) (layer "F.Cu") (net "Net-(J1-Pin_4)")))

